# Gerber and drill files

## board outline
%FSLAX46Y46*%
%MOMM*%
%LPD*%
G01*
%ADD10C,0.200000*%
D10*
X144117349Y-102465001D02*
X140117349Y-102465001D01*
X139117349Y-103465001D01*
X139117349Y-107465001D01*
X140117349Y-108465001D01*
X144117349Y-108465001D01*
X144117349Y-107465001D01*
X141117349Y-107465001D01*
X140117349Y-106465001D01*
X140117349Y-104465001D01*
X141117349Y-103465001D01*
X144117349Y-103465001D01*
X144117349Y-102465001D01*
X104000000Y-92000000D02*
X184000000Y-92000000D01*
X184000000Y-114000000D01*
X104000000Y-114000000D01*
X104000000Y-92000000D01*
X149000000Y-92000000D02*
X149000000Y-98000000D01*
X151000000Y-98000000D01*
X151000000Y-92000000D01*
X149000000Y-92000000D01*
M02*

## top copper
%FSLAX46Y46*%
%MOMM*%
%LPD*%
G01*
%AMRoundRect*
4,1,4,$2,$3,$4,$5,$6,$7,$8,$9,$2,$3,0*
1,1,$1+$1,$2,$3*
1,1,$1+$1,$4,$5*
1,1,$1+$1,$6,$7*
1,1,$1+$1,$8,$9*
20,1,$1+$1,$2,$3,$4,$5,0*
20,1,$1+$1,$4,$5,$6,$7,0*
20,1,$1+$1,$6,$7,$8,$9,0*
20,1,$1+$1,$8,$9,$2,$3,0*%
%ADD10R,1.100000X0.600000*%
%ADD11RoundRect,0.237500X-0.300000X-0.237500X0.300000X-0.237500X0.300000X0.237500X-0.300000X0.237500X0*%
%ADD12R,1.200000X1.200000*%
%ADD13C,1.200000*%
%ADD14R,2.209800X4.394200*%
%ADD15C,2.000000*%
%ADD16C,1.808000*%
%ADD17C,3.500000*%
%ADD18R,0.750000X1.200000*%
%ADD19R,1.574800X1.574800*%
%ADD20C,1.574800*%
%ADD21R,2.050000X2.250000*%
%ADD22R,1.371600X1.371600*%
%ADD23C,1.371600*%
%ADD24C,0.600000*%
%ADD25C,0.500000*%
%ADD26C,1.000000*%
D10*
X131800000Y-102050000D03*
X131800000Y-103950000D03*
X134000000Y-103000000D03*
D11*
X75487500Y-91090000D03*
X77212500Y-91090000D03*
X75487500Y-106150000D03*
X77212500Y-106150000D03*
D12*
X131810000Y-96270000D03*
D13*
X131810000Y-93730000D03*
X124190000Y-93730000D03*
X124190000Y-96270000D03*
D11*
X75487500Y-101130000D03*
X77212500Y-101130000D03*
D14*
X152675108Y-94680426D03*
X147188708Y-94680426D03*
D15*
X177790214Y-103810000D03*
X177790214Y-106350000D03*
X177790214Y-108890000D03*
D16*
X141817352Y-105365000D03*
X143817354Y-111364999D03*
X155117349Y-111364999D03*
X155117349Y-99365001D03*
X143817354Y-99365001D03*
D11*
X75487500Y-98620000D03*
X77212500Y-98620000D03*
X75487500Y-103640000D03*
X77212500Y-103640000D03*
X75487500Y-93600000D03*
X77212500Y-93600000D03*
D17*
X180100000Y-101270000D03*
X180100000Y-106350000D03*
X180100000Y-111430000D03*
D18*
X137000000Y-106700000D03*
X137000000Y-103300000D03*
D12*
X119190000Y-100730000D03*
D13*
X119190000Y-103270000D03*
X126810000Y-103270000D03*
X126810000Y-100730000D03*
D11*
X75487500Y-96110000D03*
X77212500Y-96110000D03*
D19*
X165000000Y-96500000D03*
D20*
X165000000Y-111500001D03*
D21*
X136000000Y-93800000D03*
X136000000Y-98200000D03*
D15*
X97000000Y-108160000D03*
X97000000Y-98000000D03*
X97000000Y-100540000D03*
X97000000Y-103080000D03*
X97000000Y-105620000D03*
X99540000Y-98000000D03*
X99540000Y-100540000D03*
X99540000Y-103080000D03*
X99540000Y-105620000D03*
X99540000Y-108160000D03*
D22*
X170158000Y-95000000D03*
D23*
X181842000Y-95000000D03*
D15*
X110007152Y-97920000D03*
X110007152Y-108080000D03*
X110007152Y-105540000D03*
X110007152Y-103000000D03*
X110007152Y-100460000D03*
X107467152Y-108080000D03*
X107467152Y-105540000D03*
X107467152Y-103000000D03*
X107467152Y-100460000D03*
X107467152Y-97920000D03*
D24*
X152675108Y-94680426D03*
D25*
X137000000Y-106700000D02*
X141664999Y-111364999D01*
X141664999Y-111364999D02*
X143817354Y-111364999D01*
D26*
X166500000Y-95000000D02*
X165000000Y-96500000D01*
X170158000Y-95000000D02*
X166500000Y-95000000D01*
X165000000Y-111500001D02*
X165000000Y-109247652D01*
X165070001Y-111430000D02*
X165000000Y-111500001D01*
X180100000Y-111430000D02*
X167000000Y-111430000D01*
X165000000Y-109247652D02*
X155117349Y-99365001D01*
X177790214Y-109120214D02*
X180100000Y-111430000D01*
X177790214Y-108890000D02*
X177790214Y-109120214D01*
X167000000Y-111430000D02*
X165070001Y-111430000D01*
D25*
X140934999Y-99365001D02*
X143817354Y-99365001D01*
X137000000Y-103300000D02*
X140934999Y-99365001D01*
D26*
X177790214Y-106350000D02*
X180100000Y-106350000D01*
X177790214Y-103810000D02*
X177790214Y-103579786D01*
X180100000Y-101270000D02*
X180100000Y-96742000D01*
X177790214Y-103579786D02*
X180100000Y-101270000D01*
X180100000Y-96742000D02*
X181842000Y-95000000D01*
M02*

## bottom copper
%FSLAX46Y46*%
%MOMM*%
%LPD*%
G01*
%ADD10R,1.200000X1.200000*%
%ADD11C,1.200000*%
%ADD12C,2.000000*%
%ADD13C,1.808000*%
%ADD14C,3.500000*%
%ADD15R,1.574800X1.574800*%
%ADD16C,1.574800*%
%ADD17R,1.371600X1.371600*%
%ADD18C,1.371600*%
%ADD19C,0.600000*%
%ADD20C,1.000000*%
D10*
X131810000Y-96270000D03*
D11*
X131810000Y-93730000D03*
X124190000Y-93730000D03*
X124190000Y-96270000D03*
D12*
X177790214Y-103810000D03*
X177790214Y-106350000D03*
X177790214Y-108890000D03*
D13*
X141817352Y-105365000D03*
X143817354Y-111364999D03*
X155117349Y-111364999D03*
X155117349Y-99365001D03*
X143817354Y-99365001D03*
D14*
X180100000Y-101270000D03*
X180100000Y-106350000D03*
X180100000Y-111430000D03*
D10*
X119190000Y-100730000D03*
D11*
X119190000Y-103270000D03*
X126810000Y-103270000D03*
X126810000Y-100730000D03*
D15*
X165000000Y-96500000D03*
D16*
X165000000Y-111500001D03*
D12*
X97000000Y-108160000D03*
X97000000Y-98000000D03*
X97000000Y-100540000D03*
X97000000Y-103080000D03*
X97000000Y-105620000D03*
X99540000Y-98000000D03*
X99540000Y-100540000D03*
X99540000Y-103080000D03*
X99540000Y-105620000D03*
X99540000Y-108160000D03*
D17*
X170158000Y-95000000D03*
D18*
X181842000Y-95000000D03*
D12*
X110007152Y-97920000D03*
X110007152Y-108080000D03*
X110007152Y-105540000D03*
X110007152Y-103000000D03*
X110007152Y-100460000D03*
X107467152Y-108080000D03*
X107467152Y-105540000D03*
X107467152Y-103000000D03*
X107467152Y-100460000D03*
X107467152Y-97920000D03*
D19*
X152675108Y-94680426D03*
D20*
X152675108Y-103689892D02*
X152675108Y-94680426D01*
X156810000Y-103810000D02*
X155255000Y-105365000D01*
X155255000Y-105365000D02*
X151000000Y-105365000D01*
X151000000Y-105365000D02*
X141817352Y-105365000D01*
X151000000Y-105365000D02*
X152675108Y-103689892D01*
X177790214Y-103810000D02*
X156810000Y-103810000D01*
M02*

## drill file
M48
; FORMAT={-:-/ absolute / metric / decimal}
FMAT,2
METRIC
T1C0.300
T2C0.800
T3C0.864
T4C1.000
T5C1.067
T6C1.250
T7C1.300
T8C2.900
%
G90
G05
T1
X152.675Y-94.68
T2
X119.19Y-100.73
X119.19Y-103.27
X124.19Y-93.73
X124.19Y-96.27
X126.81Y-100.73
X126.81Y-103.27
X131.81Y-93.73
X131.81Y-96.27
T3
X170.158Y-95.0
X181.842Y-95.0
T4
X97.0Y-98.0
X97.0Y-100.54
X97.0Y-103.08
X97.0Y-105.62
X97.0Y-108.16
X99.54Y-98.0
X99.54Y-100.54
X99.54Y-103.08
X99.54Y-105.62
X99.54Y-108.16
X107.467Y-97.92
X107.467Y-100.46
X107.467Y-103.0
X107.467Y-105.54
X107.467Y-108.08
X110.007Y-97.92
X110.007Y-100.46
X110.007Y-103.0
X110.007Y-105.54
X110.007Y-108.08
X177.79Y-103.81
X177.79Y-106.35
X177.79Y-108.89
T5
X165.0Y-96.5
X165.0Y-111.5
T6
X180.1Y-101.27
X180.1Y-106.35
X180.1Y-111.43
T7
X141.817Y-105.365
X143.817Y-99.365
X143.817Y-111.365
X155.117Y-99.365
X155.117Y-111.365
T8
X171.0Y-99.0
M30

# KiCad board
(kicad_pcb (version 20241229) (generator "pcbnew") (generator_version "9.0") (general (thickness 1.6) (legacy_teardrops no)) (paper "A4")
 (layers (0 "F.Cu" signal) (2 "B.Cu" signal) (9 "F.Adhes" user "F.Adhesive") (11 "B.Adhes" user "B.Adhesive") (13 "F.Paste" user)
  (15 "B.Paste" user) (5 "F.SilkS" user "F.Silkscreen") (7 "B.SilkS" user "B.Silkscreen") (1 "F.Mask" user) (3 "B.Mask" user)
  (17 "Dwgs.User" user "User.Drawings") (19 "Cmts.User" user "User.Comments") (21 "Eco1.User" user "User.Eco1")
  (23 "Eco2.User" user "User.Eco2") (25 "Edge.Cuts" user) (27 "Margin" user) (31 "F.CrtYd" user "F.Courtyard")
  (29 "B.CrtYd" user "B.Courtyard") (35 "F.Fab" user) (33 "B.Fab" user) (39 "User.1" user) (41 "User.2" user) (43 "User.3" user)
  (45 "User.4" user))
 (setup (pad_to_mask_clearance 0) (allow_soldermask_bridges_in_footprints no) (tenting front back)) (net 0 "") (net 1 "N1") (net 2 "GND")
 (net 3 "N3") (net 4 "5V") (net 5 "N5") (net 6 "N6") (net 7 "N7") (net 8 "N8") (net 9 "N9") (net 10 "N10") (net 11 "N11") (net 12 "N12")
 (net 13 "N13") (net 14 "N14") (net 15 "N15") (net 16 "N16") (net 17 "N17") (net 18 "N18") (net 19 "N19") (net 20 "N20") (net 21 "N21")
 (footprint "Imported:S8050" (layer "F.Cu") (at 132.9 103)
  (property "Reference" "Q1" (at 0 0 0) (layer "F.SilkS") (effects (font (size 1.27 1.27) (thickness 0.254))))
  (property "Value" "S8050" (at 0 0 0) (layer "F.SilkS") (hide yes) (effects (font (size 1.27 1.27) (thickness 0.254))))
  (pad "1" smd rect (at -1.1 -0.95 90) (size 0.6 1.1) (layers "F.Cu" "F.Mask" "F.Paste") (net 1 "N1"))
  (pad "2" smd rect (at -1.1 0.95 90) (size 0.6 1.1) (layers "F.Cu" "F.Mask" "F.Paste") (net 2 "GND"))
  (pad "3" smd rect (at 1.1 0 90) (size 0.6 1.1) (layers "F.Cu" "F.Mask" "F.Paste") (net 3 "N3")))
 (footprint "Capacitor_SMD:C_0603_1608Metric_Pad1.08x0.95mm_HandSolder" (layer "F.Cu") (at 76.35 91.09)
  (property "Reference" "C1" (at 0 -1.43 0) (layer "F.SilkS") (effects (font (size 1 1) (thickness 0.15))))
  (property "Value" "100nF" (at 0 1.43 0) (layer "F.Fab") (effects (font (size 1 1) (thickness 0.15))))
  (pad "1" smd roundrect (at -0.8625 0) (size 1.075 0.95) (layers "F.Cu" "F.Mask" "F.Paste") (roundrect_rratio 0.25) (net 2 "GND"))
  (pad "2" smd roundrect (at 0.8625 0) (size 1.075 0.95) (layers "F.Cu" "F.Mask" "F.Paste") (roundrect_rratio 0.25) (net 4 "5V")))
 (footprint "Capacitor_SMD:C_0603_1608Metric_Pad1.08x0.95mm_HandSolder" (layer "F.Cu") (at 76.35 106.15)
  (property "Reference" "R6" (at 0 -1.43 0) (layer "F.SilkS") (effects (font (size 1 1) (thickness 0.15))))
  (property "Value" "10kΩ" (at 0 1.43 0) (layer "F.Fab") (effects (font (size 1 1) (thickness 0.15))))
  (pad "1" smd roundrect (at -0.8625 0) (size 1.075 0.95) (layers "F.Cu" "F.Mask" "F.Paste") (roundrect_rratio 0.25) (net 2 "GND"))
  (pad "2" smd roundrect (at 0.8625 0) (size 1.075 0.95) (layers "F.Cu" "F.Mask" "F.Paste") (roundrect_rratio 0.25) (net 1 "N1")))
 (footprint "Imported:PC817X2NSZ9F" (layer "F.Cu") (at 128 95 180)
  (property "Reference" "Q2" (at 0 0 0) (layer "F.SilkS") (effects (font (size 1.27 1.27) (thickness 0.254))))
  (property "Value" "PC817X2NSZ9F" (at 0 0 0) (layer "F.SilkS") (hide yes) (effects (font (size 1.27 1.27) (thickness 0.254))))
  (pad "1" thru_hole rect (at -3.81 -1.27 180) (size 1.2 1.2) (drill 0.8) (layers "*.Cu" "*.Mask") (remove_unused_layers no) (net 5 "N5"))
  (pad "2" thru_hole circle (at -3.81 1.27 180) (size 1.2 1.2) (drill 0.8) (layers "*.Cu" "*.Mask") (remove_unused_layers no) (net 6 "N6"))
  (pad "3" thru_hole circle (at 3.81 1.27 180) (size 1.2 1.2) (drill 0.8) (layers "*.Cu" "*.Mask") (remove_unused_layers no) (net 2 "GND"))
  (pad "4" thru_hole circle (at 3.81 -1.27 180) (size 1.2 1.2) (drill 0.8) (layers "*.Cu" "*.Mask") (remove_unused_layers no) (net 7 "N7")))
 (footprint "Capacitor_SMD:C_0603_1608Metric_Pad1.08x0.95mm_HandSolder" (layer "F.Cu") (at 76.35 101.13)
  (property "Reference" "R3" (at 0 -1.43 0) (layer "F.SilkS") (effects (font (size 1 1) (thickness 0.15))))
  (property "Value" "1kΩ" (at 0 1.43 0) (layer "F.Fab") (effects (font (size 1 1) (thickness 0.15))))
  (pad "1" smd roundrect (at -0.8625 0) (size 1.075 0.95) (layers "F.Cu" "F.Mask" "F.Paste") (roundrect_rratio 0.25) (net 1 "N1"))
  (pad "2" smd roundrect (at 0.8625 0) (size 1.075 0.95) (layers "F.Cu" "F.Mask" "F.Paste") (roundrect_rratio 0.25) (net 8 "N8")))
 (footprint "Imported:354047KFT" (layer "F.Cu") (at 149.931908 94.680426 180)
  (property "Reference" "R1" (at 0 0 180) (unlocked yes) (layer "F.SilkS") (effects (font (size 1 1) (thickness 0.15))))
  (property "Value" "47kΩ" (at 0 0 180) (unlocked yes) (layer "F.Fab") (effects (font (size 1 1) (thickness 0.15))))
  (pad "1" smd rect (at -2.7432 0 180) (size 2.2098 4.3942) (layers "F.Cu" "F.Mask" "F.Paste") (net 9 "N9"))
  (pad "2" smd rect (at 2.7432 0 180) (size 2.2098 4.3942) (layers "F.Cu" "F.Mask" "F.Paste") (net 5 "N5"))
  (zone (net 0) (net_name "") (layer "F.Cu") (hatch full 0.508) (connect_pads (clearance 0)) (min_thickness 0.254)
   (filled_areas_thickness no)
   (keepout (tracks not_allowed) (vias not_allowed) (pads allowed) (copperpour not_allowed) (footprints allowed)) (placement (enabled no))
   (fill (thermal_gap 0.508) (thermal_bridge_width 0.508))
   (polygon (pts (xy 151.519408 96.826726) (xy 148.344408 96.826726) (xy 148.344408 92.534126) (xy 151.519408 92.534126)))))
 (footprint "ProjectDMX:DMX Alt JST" (layer "F.Cu") (at 177.790214 108.89 180)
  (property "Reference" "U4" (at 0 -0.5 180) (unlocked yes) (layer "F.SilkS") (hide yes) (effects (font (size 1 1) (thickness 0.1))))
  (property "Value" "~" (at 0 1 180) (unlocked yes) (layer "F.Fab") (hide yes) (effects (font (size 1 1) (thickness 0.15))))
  (pad "1" thru_hole circle (at 0 5.08 180) (size 2 2) (drill 1) (layers "*.Cu" "*.Mask") (remove_unused_layers no) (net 9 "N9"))
  (pad "2" thru_hole circle (at 0 2.54 180) (size 2 2) (drill 1) (layers "*.Cu" "*.Mask") (remove_unused_layers no) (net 6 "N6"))
  (pad "3" thru_hole circle (at 0 0 180) (size 2 2) (drill 1) (layers "*.Cu" "*.Mask") (remove_unused_layers no) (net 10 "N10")))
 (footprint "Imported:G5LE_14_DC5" (layer "F.Cu") (at 158.31735 105.365 90)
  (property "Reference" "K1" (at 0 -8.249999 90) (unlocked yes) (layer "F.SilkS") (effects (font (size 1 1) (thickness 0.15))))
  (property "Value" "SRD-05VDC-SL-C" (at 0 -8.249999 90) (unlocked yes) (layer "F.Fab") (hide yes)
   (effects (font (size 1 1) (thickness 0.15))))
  (pad "1" thru_hole circle (at 0 -16.499998 90) (size 1.808 1.808) (drill 1.3) (layers "*.Cu" "*.Mask") (remove_unused_layers no)
   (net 9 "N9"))
  (pad "2" thru_hole circle (at -5.999999 -14.499996 90) (size 1.808 1.808) (drill 1.3) (layers "*.Cu" "*.Mask") (remove_unused_layers no)
   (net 4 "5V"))
  (pad "3" thru_hole circle (at -5.999999 -3.200001 90) (size 1.808 1.808) (drill 1.3) (layers "*.Cu" "*.Mask") (remove_unused_layers no)
   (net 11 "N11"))
  (pad "4" thru_hole circle (at 5.999999 -3.200001 90) (size 1.808 1.808) (drill 1.3) (layers "*.Cu" "*.Mask") (remove_unused_layers no)
   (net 10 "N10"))
  (pad "5" thru_hole circle (at 5.999999 -14.499996 90) (size 1.808 1.808) (drill 1.3) (layers "*.Cu" "*.Mask") (remove_unused_layers no)
   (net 3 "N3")))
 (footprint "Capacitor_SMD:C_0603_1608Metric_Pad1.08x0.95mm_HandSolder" (layer "F.Cu") (at 76.35 98.62)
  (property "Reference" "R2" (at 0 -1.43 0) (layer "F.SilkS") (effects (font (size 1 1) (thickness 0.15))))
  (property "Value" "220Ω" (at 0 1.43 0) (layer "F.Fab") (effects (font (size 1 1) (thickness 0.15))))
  (pad "1" smd roundrect (at -0.8625 0) (size 1.075 0.95) (layers "F.Cu" "F.Mask" "F.Paste") (roundrect_rratio 0.25) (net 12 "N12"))
  (pad "2" smd roundrect (at 0.8625 0) (size 1.075 0.95) (layers "F.Cu" "F.Mask" "F.Paste") (roundrect_rratio 0.25) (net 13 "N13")))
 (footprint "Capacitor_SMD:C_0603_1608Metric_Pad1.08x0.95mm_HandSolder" (layer "F.Cu") (at 76.35 103.64)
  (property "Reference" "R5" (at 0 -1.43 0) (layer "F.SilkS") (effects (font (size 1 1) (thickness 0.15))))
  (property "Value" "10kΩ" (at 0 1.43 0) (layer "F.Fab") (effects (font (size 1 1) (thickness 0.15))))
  (pad "1" smd roundrect (at -0.8625 0) (size 1.075 0.95) (layers "F.Cu" "F.Mask" "F.Paste") (roundrect_rratio 0.25) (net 2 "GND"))
  (pad "2" smd roundrect (at 0.8625 0) (size 1.075 0.95) (layers "F.Cu" "F.Mask" "F.Paste") (roundrect_rratio 0.25) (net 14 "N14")))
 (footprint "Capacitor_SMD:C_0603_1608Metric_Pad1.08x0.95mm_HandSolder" (layer "F.Cu") (at 76.35 93.6)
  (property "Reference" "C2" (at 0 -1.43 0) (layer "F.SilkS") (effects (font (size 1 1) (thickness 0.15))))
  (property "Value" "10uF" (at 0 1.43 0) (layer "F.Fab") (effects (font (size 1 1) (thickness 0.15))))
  (pad "1" smd roundrect (at -0.8625 0) (size 1.075 0.95) (layers "F.Cu" "F.Mask" "F.Paste") (roundrect_rratio 0.25) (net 2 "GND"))
  (pad "2" smd roundrect (at 0.8625 0) (size 1.075 0.95) (layers "F.Cu" "F.Mask" "F.Paste") (roundrect_rratio 0.25) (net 4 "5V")))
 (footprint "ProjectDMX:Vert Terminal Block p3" (layer "F.Cu") (at 183.85 113.85 180)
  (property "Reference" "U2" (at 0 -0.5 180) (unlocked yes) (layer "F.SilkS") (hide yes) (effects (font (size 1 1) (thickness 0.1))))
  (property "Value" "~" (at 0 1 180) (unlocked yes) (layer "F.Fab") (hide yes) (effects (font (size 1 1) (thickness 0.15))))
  (pad "1" thru_hole circle (at 3.75 12.58 180) (size 3.5 3.5) (drill 1.25) (layers "*.Cu" "*.Mask") (remove_unused_layers no) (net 9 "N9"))
  (pad "2" thru_hole circle (at 3.75 7.5 180) (size 3.5 3.5) (drill 1.25) (layers "*.Cu" "*.Mask") (remove_unused_layers no) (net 6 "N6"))
  (pad "3" thru_hole circle (at 3.75 2.42 180) (size 3.5 3.5) (drill 1.25) (layers "*.Cu" "*.Mask") (remove_unused_layers no) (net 10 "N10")))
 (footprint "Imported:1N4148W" (layer "F.Cu") (at 137 105 90)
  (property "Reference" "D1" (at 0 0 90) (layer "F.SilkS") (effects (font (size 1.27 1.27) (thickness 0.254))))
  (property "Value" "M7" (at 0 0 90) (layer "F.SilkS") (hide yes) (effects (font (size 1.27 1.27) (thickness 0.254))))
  (pad "1" smd rect (at -1.7 0 180) (size 0.75 1.2) (layers "F.Cu" "F.Mask" "F.Paste") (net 4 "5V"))
  (pad "2" smd rect (at 1.7 0 180) (size 0.75 1.2) (layers "F.Cu" "F.Mask" "F.Paste") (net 3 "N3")))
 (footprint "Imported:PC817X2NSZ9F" (layer "F.Cu") (at 123 102)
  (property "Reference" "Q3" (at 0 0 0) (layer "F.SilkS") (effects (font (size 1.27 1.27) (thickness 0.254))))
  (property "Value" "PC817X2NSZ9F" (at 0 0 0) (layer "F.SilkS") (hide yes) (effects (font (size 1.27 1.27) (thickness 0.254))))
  (pad "1" thru_hole rect (at -3.81 -1.27) (size 1.2 1.2) (drill 0.8) (layers "*.Cu" "*.Mask") (remove_unused_layers no) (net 12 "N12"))
  (pad "2" thru_hole circle (at -3.81 1.27) (size 1.2 1.2) (drill 0.8) (layers "*.Cu" "*.Mask") (remove_unused_layers no) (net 2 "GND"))
  (pad "3" thru_hole circle (at 3.81 1.27) (size 1.2 1.2) (drill 0.8) (layers "*.Cu" "*.Mask") (remove_unused_layers no) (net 8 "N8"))
  (pad "4" thru_hole circle (at 3.81 -1.27) (size 1.2 1.2) (drill 0.8) (layers "*.Cu" "*.Mask") (remove_unused_layers no) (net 4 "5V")))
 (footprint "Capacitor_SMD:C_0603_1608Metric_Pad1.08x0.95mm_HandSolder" (layer "F.Cu") (at 76.35 96.11)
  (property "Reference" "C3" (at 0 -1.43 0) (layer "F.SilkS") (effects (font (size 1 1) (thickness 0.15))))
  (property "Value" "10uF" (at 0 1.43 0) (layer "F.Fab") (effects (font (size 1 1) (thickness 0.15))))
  (pad "1" smd roundrect (at -0.8625 0) (size 1.075 0.95) (layers "F.Cu" "F.Mask" "F.Paste") (roundrect_rratio 0.25) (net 7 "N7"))
  (pad "2" smd roundrect (at 0.8625 0) (size 1.075 0.95) (layers "F.Cu" "F.Mask" "F.Paste") (roundrect_rratio 0.25) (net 2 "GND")))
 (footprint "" (layer "F.Cu") (at 184 92)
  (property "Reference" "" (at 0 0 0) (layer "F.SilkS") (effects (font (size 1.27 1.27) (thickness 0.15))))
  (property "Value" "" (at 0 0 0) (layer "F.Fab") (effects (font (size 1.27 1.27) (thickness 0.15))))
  (pad "" np_thru_hole circle (at -13 7) (size 2.9 2.9) (drill 2.9) (layers "*.Cu" "*.Mask")))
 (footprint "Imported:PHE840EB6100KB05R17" (layer "F.Cu") (at 165 96.5 -90)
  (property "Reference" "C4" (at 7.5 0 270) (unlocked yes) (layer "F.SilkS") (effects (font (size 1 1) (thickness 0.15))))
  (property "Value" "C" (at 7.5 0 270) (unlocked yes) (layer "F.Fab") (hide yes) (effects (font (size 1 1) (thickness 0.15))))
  (pad "1" thru_hole rect (at 0 0 270) (size 1.5748 1.5748) (drill 1.0668) (layers "*.Cu" "*.Mask") (remove_unused_layers no) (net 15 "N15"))
  (pad "2" thru_hole circle (at 15.000001 0 270) (size 1.5748 1.5748) (drill 1.0668) (layers "*.Cu" "*.Mask") (remove_unused_layers no)
   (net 10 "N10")))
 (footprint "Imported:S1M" (layer "F.Cu") (at 136 96 -90)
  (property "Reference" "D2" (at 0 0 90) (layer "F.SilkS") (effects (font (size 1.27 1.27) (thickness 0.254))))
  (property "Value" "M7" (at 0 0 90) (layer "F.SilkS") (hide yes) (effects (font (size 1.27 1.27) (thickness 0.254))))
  (pad "1" smd rect (at -2.2 0) (size 2.05 2.25) (layers "F.Cu" "F.Mask" "F.Paste") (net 5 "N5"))
  (pad "2" smd rect (at 2.2 0) (size 2.05 2.25) (layers "F.Cu" "F.Mask" "F.Paste") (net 6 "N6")))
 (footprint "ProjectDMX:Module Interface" (layer "F.Cu") (at 97 97.90024)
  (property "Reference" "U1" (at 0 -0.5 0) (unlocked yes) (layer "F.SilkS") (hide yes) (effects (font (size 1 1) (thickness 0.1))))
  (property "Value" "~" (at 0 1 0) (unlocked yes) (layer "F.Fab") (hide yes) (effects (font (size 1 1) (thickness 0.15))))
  (pad "" thru_hole circle (at 0 10.25976 270) (size 2 2) (drill 1) (layers "*.Cu" "*.Mask") (remove_unused_layers no))
  (pad "1" thru_hole circle (at 0 0.09976 270) (size 2 2) (drill 1) (layers "*.Cu" "*.Mask") (remove_unused_layers no) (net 7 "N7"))
  (pad "2" thru_hole circle (at 0 2.63976 270) (size 2 2) (drill 1) (layers "*.Cu" "*.Mask") (remove_unused_layers no) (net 13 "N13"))
  (pad "3" thru_hole circle (at 0 5.17976 270) (size 2 2) (drill 1) (layers "*.Cu" "*.Mask") (remove_unused_layers no) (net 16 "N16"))
  (pad "4" thru_hole circle (at 0 7.71976 270) (size 2 2) (drill 1) (layers "*.Cu" "*.Mask") (remove_unused_layers no) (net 14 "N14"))
  (pad "5" thru_hole circle (at 2.54 0.09976 270) (size 2 2) (drill 1) (layers "*.Cu" "*.Mask") (remove_unused_layers no) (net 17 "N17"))
  (pad "6" thru_hole circle (at 2.54 2.63976 270) (size 2 2) (drill 1) (layers "*.Cu" "*.Mask") (remove_unused_layers no) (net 4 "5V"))
  (pad "7" thru_hole circle (at 2.54 5.17976 270) (size 2 2) (drill 1) (layers "*.Cu" "*.Mask") (remove_unused_layers no) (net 2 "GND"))
  (pad "8" thru_hole circle (at 2.54 7.71976 270) (size 2 2) (drill 1) (layers "*.Cu" "*.Mask") (remove_unused_layers no) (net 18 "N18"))
  (pad "9" thru_hole circle (at 2.54 10.25976 270) (size 2 2) (drill 1) (layers "*.Cu" "*.Mask") (remove_unused_layers no) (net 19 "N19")))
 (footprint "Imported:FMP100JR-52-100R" (layer "F.Cu") (at 170.158 95)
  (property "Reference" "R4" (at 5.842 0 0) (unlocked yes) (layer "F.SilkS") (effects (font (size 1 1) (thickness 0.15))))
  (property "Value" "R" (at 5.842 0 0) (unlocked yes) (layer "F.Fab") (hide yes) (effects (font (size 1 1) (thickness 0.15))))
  (pad "1" thru_hole rect (at 0 0) (size 1.3716 1.3716) (drill 0.8636) (layers "*.Cu" "*.Mask") (remove_unused_layers no) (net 15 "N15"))
  (pad "2" thru_hole circle (at 11.684 0) (size 1.3716 1.3716) (drill 0.8636) (layers "*.Cu" "*.Mask") (remove_unused_layers no)
   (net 9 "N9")))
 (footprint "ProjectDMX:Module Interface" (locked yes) (layer "F.Cu") (at 107.467152 97.82024)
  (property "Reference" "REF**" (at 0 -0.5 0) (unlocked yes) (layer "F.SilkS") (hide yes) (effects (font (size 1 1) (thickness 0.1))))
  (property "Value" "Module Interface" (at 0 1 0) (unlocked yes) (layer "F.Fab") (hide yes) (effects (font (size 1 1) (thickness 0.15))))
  (pad "0" thru_hole circle (at 2.54 0.09976 270) (size 2 2) (drill 1) (layers "*.Cu" "*.Mask") (remove_unused_layers no))
  (pad "1" thru_hole circle (at 2.54 10.25976 270) (size 2 2) (drill 1) (layers "*.Cu" "*.Mask") (remove_unused_layers no))
  (pad "2" thru_hole circle (at 2.54 7.71976 270) (size 2 2) (drill 1) (layers "*.Cu" "*.Mask") (remove_unused_layers no))
  (pad "3" thru_hole circle (at 2.54 5.17976 270) (size 2 2) (drill 1) (layers "*.Cu" "*.Mask") (remove_unused_layers no) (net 2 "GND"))
  (pad "4" thru_hole circle (at 2.54 2.63976 270) (size 2 2) (drill 1) (layers "*.Cu" "*.Mask") (remove_unused_layers no) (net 4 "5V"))
  (pad "5" thru_hole circle (at 0 10.25976 270) (size 2 2) (drill 1) (layers "*.Cu" "*.Mask") (remove_unused_layers no))
  (pad "6" thru_hole circle (at 0 7.71976 270) (size 2 2) (drill 1) (layers "*.Cu" "*.Mask") (remove_unused_layers no) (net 14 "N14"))
  (pad "7" thru_hole circle (at 0 5.17976 270) (size 2 2) (drill 1) (layers "*.Cu" "*.Mask") (remove_unused_layers no) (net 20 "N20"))
  (pad "8" thru_hole circle (at 0 2.63976 270) (size 2 2) (drill 1) (layers "*.Cu" "*.Mask") (remove_unused_layers no) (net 13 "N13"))
  (pad "9" thru_hole circle (at 0 0.09976 270) (size 2 2) (drill 1) (layers "*.Cu" "*.Mask") (remove_unused_layers no) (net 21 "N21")))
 (gr_poly
  (pts (xy 144.117349 102.465001) (xy 140.117349 102.465001) (xy 139.117349 103.465001) (xy 139.117349 107.465001)
   (xy 140.117349 108.465001) (xy 144.117349 108.465001) (xy 144.117349 107.465001) (xy 141.117349 107.465001) (xy 140.117349 106.465001)
   (xy 140.117349 104.465001) (xy 141.117349 103.465001) (xy 144.117349 103.465001))
  (stroke (width 0.2) (type solid)) (fill no) (layer "Edge.Cuts"))
 (gr_rect (start 104 92) (end 184 114) (stroke (width 0.2) (type default)) (fill no) (locked yes) (layer "Edge.Cuts"))
 (gr_poly (pts (xy 149 92) (xy 149 98) (xy 151 98) (xy 151 92)) (stroke (width 0.2) (type solid)) (fill no) (layer "Edge.Cuts"))
 (segment (start 137 106.7) (end 141.664999 111.364999) (width 0.5) (layer "F.Cu") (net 4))
 (segment (start 141.664999 111.364999) (end 143.817354 111.364999) (width 0.5) (layer "F.Cu") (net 4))
 (segment (start 166.5 95) (end 165 96.5) (width 1) (layer "F.Cu") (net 15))
 (segment (start 170.158 95) (end 166.5 95) (width 1) (layer "F.Cu") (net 15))
 (segment (start 165 111.500001) (end 165 109.247652) (width 1) (layer "F.Cu") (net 10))
 (segment (start 165.070001 111.43) (end 165 111.500001) (width 1) (layer "F.Cu") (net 10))
 (segment (start 180.1 111.43) (end 167 111.43) (width 1) (layer "F.Cu") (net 10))
 (segment (start 165 109.247652) (end 155.117349 99.365001) (width 1) (layer "F.Cu") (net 10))
 (segment (start 177.790214 109.120214) (end 180.1 111.43) (width 1) (layer "F.Cu") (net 10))
 (segment (start 177.790214 108.89) (end 177.790214 109.120214) (width 1) (layer "F.Cu") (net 10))
 (segment (start 167 111.43) (end 165.070001 111.43) (width 1) (layer "F.Cu") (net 10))
 (segment (start 140.934999 99.365001) (end 143.817354 99.365001) (width 0.5) (layer "F.Cu") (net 3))
 (segment (start 137 103.3) (end 140.934999 99.365001) (width 0.5) (layer "F.Cu") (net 3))
 (segment (start 177.790214 106.35) (end 180.1 106.35) (width 1) (layer "F.Cu") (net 6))
 (segment (start 177.790214 103.81) (end 177.790214 103.579786) (width 1) (layer "F.Cu") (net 9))
 (segment (start 180.1 101.27) (end 180.1 96.742) (width 1) (layer "F.Cu") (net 9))
 (segment (start 177.790214 103.579786) (end 180.1 101.27) (width 1) (layer "F.Cu") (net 9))
 (segment (start 180.1 96.742) (end 181.842 95) (width 1) (layer "F.Cu") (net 9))
 (via (at 152.675108 94.680426) (size 0.6) (drill 0.3) (layers "F.Cu" "B.Cu") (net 9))
 (segment (start 152.675108 103.689892) (end 152.675108 94.680426) (width 1) (layer "B.Cu") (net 9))
 (segment (start 156.81 103.81) (end 155.255 105.365) (width 1) (layer "B.Cu") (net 9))
 (segment (start 155.255 105.365) (end 151 105.365) (width 1) (layer "B.Cu") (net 9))
 (segment (start 151 105.365) (end 141.817352 105.365) (width 1) (layer "B.Cu") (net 9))
 (segment (start 151 105.365) (end 152.675108 103.689892) (width 1) (layer "B.Cu") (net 9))
 (segment (start 177.790214 103.81) (end 156.81 103.81) (width 1) (layer "B.Cu") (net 9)))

